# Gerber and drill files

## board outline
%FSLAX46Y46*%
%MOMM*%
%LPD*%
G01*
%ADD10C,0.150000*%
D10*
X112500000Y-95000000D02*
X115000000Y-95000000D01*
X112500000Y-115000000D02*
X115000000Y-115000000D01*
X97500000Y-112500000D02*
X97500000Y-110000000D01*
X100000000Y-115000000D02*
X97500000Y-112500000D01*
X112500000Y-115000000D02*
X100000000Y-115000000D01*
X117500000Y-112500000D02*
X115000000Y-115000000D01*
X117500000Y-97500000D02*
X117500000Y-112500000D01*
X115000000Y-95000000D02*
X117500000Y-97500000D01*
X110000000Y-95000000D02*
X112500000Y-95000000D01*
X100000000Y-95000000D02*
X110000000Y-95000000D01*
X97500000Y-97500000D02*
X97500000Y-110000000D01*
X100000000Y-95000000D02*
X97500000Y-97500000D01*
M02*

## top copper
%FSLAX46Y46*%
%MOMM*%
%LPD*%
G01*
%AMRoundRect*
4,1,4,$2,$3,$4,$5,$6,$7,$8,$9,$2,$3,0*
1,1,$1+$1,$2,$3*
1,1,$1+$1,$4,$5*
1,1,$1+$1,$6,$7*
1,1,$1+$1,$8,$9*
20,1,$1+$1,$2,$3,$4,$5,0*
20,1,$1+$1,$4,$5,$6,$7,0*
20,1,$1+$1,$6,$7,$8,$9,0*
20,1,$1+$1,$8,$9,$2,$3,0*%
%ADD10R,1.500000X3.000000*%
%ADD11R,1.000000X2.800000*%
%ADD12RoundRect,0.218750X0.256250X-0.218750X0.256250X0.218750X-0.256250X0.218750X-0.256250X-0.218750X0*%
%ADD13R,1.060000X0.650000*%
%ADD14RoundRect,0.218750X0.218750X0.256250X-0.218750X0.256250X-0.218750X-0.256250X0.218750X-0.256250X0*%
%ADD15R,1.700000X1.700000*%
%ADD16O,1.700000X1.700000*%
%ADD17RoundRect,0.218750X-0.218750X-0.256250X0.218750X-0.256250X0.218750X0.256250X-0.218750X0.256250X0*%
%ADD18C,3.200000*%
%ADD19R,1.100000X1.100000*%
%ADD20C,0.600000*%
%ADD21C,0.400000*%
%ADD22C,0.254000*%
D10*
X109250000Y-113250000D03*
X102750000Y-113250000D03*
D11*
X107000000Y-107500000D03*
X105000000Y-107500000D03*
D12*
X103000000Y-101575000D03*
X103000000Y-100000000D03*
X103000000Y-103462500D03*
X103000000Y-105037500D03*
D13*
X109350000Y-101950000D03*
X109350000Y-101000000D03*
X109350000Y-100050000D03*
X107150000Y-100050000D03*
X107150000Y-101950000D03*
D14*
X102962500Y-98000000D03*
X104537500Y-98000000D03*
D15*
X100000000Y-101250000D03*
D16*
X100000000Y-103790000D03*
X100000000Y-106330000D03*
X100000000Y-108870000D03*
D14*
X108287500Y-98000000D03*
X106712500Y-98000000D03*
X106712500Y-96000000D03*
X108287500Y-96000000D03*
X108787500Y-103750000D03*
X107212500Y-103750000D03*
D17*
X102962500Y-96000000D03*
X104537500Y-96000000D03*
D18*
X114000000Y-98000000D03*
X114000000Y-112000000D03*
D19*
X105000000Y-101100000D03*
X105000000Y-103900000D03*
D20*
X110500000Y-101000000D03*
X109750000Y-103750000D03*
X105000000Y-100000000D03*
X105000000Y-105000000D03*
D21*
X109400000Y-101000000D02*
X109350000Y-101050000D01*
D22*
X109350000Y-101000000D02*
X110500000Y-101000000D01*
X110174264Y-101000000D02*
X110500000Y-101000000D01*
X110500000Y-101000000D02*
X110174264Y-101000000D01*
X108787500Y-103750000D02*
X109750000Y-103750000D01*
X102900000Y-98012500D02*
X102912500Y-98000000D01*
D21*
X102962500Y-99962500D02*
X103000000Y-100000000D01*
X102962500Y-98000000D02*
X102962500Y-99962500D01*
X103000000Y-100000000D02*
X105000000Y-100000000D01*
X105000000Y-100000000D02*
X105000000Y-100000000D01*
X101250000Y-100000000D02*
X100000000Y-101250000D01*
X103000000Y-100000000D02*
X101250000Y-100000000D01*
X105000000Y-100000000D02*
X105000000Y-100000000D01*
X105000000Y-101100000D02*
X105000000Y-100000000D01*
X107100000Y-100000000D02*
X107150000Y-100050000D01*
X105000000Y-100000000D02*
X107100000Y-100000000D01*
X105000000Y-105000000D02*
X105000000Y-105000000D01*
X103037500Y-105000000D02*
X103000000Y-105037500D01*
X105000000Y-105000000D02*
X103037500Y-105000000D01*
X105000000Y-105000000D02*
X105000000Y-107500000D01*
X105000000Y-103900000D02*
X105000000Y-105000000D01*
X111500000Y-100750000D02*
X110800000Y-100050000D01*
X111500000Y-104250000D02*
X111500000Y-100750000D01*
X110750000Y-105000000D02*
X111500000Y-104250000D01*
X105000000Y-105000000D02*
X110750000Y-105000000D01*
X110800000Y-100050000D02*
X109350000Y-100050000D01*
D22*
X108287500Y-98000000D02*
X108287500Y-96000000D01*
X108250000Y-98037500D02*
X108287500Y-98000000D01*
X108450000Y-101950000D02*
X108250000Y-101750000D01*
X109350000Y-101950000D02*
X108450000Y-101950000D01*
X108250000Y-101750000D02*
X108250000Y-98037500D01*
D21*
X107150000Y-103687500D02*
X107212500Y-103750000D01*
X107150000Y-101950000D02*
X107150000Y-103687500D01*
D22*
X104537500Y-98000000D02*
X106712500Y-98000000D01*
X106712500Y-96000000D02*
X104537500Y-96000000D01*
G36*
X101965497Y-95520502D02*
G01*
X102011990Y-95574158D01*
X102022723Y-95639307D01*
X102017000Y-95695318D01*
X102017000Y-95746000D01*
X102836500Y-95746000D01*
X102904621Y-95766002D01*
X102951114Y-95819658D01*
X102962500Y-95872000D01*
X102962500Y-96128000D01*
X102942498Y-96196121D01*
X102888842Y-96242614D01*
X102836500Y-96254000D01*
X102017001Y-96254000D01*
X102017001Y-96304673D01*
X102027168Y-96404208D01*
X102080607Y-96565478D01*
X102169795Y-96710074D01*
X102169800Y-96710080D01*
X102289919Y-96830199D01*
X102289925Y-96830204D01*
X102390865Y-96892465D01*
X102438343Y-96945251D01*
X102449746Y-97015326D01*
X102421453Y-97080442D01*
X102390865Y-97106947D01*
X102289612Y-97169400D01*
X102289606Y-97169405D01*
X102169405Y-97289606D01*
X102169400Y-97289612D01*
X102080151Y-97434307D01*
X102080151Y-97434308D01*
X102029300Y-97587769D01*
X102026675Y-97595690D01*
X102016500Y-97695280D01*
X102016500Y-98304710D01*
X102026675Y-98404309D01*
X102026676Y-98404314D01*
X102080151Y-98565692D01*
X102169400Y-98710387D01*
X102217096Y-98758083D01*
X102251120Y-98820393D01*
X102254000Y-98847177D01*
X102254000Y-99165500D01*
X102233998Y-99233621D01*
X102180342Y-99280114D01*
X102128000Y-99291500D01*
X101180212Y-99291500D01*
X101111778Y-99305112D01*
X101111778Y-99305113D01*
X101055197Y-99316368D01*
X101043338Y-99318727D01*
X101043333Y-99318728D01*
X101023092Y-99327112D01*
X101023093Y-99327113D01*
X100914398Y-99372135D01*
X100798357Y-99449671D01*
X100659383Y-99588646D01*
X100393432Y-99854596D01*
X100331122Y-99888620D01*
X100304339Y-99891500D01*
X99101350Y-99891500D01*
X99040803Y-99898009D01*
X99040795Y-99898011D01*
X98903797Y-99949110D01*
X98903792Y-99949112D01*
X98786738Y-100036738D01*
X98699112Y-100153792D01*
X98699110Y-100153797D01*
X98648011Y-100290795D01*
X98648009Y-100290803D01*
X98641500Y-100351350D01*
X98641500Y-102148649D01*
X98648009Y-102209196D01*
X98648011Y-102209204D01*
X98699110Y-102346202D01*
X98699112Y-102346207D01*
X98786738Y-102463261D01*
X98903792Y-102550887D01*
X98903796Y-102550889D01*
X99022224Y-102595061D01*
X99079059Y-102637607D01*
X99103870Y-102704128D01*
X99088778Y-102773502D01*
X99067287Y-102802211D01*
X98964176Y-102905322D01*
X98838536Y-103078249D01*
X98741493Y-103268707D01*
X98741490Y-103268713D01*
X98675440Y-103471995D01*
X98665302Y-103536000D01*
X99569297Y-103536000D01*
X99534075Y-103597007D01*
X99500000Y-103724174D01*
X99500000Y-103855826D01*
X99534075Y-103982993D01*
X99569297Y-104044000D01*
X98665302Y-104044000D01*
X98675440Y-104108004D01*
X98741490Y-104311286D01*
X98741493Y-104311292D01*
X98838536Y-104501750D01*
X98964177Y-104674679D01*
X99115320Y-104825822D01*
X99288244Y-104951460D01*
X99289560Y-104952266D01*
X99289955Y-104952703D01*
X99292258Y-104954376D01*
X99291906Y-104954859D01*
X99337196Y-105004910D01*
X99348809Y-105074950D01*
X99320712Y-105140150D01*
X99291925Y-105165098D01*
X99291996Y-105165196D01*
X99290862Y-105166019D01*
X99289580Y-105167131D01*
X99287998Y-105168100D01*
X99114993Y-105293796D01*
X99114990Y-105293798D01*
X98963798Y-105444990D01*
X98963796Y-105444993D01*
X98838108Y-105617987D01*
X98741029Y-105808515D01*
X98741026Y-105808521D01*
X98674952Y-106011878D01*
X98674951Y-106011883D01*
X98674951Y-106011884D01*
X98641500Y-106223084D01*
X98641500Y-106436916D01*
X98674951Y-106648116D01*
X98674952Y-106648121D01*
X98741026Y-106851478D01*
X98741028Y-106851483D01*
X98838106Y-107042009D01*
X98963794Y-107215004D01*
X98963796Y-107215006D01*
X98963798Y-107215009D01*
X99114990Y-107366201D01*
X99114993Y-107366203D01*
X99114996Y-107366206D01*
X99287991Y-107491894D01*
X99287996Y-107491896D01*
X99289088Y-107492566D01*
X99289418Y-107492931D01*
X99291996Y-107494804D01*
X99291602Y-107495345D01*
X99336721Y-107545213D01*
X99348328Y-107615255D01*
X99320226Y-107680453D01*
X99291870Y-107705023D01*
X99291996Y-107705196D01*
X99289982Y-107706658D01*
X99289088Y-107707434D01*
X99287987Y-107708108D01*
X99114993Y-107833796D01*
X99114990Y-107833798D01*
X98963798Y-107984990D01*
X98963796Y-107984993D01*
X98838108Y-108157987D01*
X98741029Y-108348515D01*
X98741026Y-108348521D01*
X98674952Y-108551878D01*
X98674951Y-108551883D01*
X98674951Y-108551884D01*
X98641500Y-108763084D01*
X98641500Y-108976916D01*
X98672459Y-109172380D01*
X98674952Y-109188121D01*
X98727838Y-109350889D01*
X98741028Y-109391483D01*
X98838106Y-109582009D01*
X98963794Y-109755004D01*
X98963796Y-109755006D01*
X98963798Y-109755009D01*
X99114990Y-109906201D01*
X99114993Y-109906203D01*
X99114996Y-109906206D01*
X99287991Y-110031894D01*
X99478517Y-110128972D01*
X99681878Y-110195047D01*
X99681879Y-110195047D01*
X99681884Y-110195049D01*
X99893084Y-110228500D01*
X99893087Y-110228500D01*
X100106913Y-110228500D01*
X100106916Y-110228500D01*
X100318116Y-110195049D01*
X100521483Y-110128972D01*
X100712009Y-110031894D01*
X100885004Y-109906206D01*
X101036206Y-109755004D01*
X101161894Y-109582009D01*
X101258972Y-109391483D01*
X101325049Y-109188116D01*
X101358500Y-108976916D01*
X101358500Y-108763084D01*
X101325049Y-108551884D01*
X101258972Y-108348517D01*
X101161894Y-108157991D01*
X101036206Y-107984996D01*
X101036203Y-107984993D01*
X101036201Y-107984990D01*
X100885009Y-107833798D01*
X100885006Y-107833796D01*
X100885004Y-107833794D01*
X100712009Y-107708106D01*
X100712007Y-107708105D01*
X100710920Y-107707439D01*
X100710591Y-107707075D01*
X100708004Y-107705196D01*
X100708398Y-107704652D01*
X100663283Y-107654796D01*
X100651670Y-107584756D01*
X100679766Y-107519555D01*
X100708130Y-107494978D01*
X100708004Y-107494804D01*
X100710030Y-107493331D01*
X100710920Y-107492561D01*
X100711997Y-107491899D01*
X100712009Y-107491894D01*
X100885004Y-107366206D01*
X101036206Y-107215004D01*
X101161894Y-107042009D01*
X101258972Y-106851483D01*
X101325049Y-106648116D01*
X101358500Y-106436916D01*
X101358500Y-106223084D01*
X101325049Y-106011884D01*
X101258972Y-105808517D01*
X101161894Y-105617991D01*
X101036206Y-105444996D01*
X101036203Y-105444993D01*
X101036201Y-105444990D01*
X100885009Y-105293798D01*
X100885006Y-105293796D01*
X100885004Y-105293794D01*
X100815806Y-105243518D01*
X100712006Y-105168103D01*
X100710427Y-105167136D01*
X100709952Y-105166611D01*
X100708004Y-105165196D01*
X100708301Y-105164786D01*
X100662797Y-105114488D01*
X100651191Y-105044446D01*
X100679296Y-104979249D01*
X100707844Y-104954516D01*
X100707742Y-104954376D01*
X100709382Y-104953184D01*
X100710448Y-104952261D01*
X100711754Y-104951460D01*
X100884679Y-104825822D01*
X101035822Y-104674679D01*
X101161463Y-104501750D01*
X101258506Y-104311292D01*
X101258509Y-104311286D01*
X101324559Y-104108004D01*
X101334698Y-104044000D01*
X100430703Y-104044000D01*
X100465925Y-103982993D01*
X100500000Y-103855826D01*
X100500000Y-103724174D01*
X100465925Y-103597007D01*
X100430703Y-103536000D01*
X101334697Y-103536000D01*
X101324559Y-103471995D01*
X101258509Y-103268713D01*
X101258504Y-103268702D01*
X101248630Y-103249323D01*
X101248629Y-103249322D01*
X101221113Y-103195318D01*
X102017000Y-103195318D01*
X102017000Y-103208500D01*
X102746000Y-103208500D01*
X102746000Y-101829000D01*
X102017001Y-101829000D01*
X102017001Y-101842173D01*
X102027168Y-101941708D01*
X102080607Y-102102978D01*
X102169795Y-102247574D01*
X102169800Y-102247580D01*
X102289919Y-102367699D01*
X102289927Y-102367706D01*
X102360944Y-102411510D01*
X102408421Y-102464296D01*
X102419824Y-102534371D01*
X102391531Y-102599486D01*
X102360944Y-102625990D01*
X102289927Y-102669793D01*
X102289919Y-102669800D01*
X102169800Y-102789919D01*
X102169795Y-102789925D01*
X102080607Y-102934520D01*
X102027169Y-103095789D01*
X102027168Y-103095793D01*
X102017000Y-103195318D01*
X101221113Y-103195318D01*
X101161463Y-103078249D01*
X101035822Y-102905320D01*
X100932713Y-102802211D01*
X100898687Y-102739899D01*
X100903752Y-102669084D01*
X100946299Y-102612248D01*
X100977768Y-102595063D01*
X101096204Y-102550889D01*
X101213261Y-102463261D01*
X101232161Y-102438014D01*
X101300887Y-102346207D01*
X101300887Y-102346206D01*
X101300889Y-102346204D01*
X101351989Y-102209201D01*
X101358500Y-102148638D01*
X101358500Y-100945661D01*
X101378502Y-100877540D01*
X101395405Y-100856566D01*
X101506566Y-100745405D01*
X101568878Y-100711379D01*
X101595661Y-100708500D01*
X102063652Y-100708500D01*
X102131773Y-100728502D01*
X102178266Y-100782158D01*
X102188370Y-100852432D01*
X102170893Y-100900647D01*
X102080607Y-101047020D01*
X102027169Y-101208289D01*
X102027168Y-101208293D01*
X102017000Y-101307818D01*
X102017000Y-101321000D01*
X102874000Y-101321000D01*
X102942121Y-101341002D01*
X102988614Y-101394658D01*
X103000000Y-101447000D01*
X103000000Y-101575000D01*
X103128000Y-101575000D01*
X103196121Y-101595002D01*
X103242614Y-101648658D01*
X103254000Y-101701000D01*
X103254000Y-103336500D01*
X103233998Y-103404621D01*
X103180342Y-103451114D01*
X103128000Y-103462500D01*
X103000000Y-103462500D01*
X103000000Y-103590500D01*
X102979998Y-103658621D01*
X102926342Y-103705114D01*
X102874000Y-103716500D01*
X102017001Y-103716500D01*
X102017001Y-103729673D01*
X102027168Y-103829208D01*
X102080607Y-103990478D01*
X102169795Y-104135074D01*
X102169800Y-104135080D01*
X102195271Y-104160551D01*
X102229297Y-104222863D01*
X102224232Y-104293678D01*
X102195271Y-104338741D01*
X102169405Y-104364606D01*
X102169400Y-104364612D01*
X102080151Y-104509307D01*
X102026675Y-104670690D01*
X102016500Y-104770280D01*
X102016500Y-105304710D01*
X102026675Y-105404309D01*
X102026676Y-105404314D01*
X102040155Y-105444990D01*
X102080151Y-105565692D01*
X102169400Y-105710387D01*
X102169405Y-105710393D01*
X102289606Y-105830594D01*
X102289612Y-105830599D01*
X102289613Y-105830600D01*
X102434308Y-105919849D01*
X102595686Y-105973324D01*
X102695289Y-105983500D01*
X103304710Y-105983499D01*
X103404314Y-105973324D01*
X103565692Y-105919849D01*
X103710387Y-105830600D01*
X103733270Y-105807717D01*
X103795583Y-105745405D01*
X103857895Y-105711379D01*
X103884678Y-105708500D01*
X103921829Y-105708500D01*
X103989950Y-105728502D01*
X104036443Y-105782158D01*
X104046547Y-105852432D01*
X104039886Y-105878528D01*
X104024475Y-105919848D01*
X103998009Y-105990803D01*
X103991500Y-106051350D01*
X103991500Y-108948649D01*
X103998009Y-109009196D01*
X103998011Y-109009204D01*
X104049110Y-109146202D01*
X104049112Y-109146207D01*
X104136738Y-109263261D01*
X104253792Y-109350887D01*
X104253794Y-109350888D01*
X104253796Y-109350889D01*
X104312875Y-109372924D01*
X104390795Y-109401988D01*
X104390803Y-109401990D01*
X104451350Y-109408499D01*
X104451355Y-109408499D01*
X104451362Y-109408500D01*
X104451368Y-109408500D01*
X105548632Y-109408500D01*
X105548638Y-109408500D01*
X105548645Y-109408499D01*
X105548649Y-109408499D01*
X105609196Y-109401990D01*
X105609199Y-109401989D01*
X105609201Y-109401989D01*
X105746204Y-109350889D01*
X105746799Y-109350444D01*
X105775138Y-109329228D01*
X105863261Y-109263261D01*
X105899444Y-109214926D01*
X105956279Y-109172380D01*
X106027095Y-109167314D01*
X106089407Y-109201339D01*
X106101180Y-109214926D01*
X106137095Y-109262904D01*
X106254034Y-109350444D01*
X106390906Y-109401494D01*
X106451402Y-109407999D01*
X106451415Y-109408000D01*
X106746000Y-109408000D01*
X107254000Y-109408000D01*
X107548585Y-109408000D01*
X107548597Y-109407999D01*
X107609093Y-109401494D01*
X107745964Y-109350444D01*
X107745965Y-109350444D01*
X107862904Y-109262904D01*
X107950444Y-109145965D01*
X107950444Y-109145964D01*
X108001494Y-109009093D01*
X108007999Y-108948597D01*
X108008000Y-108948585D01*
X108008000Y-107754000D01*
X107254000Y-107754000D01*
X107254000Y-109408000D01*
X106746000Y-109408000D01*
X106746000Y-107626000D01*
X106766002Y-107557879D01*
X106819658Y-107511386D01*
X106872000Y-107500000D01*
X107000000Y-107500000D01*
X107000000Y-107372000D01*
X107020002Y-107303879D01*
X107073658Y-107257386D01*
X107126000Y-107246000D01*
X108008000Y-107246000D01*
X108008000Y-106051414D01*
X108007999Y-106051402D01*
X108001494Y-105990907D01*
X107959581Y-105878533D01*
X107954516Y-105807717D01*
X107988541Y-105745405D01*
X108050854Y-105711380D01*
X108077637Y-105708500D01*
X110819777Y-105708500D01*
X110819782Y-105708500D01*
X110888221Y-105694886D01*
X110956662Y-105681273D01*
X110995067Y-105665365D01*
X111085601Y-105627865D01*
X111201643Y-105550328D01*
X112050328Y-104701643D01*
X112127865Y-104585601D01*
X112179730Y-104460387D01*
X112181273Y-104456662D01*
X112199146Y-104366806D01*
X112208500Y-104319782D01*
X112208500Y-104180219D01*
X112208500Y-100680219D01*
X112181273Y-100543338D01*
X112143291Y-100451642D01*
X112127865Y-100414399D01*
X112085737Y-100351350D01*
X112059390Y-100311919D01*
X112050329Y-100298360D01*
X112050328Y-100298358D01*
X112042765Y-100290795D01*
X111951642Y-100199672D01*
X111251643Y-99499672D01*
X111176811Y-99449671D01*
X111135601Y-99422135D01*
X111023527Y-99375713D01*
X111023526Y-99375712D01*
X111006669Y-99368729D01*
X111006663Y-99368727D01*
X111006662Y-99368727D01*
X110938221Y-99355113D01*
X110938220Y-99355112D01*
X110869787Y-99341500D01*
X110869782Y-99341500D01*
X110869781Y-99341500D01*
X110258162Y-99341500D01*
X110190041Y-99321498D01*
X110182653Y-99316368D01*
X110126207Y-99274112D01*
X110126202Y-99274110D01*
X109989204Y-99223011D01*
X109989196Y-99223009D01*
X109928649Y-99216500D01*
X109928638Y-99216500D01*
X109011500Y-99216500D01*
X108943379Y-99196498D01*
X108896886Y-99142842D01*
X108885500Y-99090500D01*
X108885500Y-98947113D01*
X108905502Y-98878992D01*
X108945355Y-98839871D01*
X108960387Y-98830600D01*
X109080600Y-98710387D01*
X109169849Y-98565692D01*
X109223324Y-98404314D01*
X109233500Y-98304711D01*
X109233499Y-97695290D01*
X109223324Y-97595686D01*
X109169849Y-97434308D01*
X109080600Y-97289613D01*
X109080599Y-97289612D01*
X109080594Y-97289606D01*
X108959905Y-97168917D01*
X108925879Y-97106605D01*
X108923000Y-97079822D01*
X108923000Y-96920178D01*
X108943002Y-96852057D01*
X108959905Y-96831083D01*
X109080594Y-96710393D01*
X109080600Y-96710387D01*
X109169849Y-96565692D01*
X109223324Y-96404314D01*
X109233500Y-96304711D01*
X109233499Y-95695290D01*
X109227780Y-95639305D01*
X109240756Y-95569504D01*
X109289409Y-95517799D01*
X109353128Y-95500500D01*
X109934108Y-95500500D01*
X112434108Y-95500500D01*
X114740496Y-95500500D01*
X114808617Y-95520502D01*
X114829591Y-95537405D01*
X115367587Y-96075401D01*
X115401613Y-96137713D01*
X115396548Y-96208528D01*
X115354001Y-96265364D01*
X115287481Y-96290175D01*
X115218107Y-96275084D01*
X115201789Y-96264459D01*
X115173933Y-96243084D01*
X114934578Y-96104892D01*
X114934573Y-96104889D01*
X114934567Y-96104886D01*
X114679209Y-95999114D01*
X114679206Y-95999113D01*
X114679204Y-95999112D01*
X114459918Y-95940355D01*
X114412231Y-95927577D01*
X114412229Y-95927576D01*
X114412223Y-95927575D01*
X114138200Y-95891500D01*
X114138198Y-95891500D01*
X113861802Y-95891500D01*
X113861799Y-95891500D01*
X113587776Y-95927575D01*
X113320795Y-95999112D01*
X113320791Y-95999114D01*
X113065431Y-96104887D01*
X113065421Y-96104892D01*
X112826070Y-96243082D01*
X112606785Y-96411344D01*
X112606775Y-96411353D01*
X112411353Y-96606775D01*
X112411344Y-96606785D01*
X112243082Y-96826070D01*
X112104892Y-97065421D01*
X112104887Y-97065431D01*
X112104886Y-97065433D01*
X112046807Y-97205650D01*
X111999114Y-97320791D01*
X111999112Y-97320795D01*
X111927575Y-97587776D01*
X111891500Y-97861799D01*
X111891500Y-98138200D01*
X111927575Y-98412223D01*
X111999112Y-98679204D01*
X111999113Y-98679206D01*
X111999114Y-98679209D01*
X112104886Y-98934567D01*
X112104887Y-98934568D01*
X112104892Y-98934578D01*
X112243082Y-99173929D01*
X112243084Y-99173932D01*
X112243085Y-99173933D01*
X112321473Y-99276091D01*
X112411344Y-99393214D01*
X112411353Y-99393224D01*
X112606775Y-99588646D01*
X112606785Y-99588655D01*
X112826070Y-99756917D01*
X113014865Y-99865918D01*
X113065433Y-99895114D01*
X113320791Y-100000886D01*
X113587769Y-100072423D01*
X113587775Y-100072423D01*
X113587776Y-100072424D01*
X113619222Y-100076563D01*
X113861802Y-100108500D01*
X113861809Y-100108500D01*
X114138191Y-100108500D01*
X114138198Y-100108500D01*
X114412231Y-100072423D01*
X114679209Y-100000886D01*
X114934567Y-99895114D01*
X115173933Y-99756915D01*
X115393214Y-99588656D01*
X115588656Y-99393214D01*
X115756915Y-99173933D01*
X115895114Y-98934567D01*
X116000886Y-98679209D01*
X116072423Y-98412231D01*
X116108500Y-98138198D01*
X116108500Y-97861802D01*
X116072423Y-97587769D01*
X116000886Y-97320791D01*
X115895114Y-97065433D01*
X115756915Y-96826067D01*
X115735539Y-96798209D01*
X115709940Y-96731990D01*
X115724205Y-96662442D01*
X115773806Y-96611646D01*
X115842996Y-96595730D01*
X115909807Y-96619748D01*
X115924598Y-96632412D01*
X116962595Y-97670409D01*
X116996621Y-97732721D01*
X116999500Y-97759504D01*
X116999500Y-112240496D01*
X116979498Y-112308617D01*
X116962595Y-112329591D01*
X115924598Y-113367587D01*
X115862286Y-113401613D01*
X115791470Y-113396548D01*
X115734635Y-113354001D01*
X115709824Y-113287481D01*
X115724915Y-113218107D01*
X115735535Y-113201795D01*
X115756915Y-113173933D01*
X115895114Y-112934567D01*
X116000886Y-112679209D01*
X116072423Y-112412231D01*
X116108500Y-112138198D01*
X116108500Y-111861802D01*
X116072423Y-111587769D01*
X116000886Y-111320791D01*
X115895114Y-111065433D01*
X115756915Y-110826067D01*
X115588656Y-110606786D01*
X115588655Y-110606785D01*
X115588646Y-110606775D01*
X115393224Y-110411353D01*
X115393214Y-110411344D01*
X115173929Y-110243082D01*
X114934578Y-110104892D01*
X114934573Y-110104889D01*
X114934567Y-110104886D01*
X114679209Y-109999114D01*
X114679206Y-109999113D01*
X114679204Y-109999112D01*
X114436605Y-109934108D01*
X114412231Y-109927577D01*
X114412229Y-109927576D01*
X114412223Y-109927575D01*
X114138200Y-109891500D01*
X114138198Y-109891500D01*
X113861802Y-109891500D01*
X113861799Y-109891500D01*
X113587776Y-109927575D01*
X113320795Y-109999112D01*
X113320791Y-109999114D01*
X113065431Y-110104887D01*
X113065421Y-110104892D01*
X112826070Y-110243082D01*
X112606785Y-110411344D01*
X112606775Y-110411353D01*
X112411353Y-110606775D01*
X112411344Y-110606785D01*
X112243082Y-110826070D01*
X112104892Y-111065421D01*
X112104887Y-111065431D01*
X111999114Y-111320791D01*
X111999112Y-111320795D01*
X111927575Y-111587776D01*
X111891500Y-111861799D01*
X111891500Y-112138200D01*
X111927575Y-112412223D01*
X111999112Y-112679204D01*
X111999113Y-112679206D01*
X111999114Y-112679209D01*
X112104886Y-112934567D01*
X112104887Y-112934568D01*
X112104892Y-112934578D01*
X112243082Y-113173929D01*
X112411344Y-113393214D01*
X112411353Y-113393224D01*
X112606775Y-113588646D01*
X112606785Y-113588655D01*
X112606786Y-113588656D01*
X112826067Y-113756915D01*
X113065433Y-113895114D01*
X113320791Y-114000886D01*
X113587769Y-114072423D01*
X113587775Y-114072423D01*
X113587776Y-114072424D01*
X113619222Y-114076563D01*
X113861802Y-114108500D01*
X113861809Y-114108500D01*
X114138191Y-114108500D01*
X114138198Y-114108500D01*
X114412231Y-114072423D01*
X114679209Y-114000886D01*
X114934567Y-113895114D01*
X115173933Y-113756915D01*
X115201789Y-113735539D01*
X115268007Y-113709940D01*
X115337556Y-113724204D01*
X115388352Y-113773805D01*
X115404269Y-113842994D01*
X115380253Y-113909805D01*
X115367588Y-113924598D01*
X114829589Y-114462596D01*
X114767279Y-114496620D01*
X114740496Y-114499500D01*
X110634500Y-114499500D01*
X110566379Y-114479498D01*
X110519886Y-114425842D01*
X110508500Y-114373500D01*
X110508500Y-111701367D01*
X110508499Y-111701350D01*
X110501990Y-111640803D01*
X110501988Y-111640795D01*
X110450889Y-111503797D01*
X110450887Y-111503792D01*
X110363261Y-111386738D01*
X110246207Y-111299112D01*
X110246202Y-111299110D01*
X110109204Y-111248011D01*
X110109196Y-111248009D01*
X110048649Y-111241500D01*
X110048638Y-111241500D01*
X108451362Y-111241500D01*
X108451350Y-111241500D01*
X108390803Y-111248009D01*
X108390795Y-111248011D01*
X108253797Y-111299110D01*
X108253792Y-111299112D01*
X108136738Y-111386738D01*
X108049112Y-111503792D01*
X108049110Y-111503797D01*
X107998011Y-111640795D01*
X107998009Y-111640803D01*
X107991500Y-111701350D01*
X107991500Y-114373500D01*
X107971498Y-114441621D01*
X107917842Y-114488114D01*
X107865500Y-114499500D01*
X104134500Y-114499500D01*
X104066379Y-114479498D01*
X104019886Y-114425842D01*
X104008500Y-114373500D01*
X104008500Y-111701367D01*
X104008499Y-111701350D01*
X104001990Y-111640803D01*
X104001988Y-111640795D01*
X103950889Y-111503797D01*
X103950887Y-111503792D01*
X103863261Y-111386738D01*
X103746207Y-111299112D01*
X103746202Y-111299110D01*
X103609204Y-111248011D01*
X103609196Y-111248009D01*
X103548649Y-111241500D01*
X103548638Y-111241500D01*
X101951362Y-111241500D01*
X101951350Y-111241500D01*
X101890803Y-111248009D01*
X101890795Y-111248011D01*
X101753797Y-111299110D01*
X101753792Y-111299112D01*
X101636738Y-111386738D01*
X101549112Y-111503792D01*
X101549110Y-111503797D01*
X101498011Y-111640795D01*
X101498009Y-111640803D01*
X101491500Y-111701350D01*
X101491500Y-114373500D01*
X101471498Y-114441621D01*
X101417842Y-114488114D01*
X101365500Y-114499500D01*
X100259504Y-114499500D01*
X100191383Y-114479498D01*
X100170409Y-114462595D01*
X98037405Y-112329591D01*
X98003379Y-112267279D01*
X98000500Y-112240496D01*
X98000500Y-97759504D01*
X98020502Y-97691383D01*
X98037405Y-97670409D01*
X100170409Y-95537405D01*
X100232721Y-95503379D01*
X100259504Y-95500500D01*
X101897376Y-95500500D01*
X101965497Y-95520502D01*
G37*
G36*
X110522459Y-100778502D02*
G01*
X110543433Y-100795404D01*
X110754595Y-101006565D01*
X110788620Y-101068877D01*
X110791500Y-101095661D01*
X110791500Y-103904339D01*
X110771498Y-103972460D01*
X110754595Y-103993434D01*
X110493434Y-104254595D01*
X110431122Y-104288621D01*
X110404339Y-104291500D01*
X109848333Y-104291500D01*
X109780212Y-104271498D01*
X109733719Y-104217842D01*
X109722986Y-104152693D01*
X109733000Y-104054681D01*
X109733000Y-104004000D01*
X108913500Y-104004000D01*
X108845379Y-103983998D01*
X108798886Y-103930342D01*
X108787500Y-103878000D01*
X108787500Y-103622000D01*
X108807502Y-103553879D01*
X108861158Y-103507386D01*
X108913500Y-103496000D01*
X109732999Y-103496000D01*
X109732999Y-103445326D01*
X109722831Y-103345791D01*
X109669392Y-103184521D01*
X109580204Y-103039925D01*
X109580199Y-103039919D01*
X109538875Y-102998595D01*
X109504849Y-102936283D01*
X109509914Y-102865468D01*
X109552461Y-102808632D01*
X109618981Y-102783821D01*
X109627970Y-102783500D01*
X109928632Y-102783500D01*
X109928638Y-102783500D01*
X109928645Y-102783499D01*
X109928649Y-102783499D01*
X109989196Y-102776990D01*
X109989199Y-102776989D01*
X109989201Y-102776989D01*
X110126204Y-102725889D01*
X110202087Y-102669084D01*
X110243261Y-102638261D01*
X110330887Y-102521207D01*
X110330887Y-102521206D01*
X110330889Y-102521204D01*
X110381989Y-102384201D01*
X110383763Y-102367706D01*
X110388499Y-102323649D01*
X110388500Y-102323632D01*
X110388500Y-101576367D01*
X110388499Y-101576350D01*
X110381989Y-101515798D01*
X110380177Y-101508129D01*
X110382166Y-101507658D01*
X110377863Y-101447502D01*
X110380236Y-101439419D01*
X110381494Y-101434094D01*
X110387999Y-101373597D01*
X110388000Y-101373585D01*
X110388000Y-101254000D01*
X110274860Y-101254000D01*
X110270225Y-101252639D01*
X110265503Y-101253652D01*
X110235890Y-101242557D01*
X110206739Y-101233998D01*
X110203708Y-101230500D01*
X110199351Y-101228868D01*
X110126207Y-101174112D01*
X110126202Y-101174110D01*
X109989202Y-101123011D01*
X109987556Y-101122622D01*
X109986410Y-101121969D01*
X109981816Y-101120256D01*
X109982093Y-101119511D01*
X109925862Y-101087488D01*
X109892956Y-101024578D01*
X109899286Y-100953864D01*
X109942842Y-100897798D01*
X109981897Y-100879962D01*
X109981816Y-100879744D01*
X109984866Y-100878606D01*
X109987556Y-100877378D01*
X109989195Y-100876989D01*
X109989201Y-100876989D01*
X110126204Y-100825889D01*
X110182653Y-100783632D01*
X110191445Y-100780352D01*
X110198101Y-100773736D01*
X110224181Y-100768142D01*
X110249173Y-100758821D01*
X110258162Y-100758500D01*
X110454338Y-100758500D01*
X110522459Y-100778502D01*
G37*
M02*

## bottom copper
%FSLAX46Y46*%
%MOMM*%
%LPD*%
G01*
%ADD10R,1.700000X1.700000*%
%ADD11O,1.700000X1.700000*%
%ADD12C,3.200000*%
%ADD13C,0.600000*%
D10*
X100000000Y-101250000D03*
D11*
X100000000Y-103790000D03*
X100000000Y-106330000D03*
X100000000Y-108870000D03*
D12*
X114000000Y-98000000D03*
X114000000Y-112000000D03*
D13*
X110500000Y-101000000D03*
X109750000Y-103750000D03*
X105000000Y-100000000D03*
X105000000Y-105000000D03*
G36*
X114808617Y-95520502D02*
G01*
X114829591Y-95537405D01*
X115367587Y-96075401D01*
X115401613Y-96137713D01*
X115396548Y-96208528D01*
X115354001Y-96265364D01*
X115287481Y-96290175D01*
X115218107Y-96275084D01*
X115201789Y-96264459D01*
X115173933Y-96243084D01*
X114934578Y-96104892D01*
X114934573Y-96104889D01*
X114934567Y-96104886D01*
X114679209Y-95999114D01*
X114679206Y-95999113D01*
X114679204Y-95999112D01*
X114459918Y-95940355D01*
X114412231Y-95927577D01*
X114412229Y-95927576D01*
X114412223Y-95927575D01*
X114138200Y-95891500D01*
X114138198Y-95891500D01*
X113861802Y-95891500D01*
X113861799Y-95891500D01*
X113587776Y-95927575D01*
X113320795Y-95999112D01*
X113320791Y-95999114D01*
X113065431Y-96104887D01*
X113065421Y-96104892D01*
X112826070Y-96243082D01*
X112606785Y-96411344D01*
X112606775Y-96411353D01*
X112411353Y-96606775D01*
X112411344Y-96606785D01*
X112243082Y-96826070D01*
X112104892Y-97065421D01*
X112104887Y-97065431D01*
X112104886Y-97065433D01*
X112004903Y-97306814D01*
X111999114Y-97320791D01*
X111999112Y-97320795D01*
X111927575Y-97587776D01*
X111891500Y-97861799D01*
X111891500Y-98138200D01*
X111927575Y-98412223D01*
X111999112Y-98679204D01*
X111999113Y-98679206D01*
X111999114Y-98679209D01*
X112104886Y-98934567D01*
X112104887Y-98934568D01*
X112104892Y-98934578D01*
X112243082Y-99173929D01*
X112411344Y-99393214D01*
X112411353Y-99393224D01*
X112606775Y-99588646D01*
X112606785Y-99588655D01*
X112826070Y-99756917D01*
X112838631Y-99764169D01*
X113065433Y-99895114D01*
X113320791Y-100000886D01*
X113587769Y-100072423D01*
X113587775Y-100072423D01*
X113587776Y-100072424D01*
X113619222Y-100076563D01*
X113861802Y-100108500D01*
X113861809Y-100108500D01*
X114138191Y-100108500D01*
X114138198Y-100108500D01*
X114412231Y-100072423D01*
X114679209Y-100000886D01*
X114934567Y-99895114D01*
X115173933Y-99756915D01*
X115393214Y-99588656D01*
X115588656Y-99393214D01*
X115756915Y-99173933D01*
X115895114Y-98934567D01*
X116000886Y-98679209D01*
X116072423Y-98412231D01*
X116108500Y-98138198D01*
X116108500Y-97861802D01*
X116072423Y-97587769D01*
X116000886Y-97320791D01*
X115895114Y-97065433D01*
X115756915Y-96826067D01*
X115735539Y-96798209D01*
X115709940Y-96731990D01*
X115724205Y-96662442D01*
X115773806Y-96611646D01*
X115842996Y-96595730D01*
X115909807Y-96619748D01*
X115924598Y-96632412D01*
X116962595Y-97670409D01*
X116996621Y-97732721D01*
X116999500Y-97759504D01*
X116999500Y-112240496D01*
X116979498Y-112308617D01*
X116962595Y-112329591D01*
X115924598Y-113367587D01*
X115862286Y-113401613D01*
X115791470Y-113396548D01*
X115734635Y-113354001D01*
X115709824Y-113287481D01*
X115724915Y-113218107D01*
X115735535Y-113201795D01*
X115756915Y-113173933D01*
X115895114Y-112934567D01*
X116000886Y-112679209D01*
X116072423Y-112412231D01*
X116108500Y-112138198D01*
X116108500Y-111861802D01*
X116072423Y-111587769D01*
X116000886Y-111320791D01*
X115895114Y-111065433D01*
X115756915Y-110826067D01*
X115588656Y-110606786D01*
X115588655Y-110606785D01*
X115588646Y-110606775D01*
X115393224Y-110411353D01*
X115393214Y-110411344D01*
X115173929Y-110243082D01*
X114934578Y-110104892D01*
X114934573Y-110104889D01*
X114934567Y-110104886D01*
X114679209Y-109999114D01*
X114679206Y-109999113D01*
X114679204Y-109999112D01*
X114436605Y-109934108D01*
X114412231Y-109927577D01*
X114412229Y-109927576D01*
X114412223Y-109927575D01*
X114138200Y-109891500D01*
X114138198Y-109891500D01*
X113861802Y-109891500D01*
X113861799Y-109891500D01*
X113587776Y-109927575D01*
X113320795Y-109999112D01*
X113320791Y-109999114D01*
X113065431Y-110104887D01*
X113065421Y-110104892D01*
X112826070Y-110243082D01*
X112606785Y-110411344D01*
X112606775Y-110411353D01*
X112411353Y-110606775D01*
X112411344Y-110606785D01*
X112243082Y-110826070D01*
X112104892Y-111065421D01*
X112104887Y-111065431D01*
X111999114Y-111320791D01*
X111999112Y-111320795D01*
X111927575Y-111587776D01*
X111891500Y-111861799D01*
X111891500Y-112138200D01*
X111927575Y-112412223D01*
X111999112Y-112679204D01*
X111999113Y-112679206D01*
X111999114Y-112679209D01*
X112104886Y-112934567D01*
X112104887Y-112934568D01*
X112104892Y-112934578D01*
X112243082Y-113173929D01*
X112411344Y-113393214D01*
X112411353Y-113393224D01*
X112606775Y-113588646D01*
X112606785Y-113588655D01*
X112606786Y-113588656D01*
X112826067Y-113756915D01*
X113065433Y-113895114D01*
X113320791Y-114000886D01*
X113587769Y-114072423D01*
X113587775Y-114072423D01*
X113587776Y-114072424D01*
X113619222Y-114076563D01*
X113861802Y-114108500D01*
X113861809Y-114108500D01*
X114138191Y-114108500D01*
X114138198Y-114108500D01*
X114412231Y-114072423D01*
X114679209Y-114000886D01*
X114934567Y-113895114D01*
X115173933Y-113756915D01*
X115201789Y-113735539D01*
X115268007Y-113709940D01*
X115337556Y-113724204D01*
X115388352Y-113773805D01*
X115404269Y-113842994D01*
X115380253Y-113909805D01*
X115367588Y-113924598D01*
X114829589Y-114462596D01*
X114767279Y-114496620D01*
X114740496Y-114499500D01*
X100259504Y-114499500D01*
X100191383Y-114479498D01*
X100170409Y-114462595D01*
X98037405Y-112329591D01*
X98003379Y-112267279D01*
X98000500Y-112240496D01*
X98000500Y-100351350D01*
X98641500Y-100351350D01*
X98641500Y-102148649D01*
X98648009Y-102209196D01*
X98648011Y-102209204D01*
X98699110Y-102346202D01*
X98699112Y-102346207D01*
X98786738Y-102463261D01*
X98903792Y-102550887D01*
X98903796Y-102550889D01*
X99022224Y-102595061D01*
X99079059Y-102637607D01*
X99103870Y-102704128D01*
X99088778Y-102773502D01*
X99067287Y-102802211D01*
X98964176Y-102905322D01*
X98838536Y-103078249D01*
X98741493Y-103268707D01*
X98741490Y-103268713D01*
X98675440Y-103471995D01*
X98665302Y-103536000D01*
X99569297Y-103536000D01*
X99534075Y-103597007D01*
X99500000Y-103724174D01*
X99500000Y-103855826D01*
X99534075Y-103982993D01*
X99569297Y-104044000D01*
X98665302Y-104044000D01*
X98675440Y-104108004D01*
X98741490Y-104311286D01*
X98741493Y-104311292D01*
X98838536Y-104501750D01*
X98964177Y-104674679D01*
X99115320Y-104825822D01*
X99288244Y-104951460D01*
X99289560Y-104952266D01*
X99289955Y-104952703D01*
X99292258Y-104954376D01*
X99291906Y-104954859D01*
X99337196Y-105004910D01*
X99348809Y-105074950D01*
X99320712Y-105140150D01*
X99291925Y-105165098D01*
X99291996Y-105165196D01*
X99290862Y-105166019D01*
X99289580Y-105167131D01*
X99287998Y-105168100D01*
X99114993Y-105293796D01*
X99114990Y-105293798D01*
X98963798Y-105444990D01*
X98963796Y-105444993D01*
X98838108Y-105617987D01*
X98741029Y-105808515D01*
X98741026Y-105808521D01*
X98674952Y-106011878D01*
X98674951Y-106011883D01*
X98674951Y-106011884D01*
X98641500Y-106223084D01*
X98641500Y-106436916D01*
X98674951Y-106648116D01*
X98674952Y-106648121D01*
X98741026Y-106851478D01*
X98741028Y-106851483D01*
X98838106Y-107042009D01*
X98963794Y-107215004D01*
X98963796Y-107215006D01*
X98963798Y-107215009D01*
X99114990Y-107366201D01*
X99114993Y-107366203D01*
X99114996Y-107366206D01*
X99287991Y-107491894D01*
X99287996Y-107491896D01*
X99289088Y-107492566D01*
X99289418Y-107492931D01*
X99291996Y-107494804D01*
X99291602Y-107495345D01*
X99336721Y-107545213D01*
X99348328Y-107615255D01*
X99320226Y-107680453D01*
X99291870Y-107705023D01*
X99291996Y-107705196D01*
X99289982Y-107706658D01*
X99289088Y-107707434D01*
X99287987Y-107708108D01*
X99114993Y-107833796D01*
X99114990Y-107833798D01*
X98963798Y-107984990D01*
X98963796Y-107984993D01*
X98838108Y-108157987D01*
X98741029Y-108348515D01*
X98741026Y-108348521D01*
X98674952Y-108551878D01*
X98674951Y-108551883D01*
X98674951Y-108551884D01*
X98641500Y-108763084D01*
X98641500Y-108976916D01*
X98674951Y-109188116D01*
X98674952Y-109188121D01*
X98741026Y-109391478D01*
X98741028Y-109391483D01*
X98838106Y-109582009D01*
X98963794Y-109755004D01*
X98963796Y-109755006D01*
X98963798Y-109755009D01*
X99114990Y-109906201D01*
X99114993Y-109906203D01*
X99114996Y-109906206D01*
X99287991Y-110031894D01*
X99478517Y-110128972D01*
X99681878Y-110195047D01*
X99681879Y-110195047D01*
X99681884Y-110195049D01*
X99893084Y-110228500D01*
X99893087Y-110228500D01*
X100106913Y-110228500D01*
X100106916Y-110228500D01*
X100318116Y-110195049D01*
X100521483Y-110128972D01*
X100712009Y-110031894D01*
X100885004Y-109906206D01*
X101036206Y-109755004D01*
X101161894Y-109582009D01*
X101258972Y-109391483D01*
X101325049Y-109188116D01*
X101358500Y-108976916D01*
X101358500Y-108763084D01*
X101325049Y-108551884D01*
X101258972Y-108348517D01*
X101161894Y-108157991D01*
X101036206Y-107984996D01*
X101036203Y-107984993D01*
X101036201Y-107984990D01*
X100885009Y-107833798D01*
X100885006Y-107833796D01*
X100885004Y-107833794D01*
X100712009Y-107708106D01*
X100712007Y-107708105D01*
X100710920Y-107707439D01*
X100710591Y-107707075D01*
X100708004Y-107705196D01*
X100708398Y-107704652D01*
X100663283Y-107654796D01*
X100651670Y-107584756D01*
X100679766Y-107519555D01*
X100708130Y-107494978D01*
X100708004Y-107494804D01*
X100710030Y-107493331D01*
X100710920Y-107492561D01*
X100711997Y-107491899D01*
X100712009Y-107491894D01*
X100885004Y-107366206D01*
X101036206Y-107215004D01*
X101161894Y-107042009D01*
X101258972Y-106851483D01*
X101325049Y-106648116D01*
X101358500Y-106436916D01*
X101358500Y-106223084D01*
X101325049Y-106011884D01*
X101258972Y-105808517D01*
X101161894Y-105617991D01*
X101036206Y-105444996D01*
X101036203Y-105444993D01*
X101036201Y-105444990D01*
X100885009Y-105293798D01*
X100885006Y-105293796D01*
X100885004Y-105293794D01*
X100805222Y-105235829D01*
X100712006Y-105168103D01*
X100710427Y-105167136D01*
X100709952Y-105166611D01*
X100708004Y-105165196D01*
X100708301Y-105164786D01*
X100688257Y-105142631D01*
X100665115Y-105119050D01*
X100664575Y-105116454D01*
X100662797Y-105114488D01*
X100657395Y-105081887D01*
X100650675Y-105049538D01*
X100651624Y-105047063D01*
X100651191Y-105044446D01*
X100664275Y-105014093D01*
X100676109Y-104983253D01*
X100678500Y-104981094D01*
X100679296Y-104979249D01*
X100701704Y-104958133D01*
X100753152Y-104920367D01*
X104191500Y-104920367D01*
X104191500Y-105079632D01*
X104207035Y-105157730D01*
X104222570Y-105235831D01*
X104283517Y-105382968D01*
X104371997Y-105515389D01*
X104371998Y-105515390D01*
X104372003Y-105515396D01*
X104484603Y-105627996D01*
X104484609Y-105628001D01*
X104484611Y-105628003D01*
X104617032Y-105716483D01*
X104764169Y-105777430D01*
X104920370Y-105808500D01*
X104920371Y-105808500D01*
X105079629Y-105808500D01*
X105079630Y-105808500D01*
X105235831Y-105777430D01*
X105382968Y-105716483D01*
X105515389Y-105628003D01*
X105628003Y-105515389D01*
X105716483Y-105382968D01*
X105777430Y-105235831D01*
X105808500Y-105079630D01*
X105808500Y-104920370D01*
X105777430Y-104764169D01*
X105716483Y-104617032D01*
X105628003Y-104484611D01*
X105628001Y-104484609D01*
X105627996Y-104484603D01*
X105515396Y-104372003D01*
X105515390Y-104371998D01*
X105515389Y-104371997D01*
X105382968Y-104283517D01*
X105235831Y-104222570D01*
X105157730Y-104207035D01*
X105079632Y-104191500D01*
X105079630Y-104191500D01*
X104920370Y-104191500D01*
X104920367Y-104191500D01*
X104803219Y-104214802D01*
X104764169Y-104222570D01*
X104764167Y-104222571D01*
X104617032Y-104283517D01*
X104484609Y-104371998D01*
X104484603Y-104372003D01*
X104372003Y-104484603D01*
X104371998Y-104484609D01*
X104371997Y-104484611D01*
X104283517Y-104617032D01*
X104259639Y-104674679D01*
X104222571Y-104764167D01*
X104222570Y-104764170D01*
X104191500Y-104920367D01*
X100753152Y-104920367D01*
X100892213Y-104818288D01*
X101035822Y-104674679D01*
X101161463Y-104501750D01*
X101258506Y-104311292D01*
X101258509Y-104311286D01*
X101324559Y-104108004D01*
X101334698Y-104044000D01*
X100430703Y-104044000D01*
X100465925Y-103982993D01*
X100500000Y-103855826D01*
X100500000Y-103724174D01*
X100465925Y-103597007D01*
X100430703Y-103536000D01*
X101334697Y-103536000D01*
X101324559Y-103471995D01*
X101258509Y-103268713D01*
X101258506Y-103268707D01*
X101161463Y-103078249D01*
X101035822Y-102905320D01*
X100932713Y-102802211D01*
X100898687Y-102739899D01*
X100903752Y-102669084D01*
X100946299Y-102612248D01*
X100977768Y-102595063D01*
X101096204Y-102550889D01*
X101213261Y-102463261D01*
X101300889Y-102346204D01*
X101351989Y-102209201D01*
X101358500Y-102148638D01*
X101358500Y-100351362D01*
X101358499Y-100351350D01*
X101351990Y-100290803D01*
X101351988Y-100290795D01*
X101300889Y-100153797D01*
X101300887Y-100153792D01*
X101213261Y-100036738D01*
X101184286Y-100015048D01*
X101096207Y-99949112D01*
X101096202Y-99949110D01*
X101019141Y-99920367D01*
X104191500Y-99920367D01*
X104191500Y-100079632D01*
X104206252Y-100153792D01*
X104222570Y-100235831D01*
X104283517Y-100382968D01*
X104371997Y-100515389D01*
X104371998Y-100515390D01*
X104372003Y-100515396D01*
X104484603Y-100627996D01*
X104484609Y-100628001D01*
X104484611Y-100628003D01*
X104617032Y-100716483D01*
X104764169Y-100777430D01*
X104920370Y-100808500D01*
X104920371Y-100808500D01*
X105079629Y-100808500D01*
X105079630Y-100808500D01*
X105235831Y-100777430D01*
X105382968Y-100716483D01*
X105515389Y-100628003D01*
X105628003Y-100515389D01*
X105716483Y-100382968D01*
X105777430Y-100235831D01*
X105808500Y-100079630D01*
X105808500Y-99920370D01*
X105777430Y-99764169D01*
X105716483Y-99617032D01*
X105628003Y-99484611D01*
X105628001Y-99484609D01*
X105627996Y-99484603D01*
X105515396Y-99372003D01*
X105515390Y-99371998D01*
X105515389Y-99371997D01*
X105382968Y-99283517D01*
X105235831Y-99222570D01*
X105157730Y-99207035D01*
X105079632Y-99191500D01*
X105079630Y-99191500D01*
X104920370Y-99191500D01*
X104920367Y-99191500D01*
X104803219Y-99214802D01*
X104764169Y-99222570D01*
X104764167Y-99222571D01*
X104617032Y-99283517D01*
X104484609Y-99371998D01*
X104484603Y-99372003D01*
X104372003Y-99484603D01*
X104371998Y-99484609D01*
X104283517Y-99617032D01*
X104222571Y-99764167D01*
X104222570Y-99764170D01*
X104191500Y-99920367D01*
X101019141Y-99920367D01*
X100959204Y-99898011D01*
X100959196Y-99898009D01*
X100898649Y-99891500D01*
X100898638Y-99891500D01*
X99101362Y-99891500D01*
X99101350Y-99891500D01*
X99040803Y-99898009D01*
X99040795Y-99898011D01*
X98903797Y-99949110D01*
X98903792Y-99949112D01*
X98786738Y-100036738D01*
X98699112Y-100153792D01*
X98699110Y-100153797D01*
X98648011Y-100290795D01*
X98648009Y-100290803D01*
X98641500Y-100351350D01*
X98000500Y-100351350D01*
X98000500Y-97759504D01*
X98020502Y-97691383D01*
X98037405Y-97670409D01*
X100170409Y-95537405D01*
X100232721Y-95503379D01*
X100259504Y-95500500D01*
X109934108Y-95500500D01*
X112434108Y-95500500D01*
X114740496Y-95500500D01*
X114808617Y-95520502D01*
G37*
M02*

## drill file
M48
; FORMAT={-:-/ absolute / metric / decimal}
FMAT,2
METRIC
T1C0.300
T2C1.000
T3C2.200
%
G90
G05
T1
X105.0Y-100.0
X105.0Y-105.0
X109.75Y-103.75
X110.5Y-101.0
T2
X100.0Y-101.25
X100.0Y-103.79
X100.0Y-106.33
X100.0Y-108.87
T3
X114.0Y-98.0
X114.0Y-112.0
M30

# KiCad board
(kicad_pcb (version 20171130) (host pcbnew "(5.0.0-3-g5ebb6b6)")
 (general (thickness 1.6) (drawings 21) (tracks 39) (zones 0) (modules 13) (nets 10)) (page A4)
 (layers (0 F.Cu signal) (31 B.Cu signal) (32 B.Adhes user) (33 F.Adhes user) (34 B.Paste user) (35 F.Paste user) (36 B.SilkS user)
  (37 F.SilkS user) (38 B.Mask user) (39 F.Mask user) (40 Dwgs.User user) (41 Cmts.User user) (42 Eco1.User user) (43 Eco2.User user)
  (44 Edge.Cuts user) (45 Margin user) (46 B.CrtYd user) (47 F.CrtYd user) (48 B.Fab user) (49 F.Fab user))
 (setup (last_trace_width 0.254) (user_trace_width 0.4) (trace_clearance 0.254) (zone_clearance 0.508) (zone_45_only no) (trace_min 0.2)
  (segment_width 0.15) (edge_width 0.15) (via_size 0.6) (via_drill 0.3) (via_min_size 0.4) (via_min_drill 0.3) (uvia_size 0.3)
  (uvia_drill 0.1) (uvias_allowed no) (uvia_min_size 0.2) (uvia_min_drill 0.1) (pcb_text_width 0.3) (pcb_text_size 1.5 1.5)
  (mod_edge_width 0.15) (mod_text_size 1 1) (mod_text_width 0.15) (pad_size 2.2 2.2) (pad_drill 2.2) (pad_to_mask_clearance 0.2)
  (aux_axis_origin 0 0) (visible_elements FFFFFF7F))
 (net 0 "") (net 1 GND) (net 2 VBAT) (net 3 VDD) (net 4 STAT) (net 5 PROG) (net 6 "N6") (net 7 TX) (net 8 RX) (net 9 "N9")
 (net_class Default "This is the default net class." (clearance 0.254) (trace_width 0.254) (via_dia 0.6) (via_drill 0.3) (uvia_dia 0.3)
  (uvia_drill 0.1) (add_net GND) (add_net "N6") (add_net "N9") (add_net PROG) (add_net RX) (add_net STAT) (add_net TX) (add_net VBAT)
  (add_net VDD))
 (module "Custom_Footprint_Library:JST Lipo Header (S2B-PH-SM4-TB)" (layer F.Cu) (at 106 112)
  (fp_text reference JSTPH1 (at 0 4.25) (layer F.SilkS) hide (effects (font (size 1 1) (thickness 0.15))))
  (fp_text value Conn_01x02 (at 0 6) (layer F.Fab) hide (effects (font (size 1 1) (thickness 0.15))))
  (pad "" connect rect (at 3.25 1.25) (size 1.5 3) (layers F.Cu F.Mask))
  (pad "" connect rect (at -3.25 1.25) (size 1.5 3) (layers F.Cu F.Mask))
  (pad 2 smd rect (at 1 -4.5) (size 1 2.8) (layers F.Cu F.Paste F.Mask) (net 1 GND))
  (pad 1 smd rect (at -1 -4.5) (size 1 2.8) (layers F.Cu F.Paste F.Mask) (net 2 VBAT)))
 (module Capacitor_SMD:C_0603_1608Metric (layer F.Cu) (at 103 100.7875 90)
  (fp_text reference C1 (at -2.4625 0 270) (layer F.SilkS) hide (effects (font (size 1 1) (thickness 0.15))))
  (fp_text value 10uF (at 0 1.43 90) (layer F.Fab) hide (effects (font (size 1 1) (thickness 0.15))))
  (pad 1 smd roundrect (at -0.7875 0 90) (size 0.875 0.95) (layers F.Cu F.Paste F.Mask) (roundrect_rratio 0.25) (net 1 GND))
  (pad 2 smd roundrect (at 0.7875 0 90) (size 0.875 0.95) (layers F.Cu F.Paste F.Mask) (roundrect_rratio 0.25) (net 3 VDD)))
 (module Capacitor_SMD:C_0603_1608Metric (layer F.Cu) (at 103 104.25 90)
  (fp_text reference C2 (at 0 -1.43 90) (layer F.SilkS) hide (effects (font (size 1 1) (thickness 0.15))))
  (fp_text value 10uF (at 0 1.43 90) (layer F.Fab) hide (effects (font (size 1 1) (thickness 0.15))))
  (pad 2 smd roundrect (at 0.7875 0 90) (size 0.875 0.95) (layers F.Cu F.Paste F.Mask) (roundrect_rratio 0.25) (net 1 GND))
  (pad 1 smd roundrect (at -0.7875 0 90) (size 0.875 0.95) (layers F.Cu F.Paste F.Mask) (roundrect_rratio 0.25) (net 2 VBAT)))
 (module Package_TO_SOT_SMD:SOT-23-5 (layer F.Cu) (at 108.25 101 180)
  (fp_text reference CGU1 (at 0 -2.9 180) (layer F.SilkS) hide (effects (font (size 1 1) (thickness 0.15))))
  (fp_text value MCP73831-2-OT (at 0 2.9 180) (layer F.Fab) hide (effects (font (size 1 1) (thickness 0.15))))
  (pad 1 smd rect (at -1.1 -0.95 180) (size 1.06 0.65) (layers F.Cu F.Paste F.Mask) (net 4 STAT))
  (pad 2 smd rect (at -1.1 0 180) (size 1.06 0.65) (layers F.Cu F.Paste F.Mask) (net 1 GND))
  (pad 3 smd rect (at -1.1 0.95 180) (size 1.06 0.65) (layers F.Cu F.Paste F.Mask) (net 2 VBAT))
  (pad 4 smd rect (at 1.1 0.95 180) (size 1.06 0.65) (layers F.Cu F.Paste F.Mask) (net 3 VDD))
  (pad 5 smd rect (at 1.1 -0.95 180) (size 1.06 0.65) (layers F.Cu F.Paste F.Mask) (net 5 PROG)))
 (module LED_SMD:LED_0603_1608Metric (layer F.Cu) (at 103.75 98 180)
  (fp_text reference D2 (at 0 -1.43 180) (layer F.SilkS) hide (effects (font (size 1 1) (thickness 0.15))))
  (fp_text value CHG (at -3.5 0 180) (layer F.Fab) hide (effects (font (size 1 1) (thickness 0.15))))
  (pad 2 smd roundrect (at 0.7875 0 180) (size 0.875 0.95) (layers F.Cu F.Paste F.Mask) (roundrect_rratio 0.25) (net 3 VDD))
  (pad 1 smd roundrect (at -0.7875 0 180) (size 0.875 0.95) (layers F.Cu F.Paste F.Mask) (roundrect_rratio 0.25) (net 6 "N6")))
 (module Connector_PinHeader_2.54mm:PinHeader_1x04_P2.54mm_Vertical (layer F.Cu) (at 100 101.25)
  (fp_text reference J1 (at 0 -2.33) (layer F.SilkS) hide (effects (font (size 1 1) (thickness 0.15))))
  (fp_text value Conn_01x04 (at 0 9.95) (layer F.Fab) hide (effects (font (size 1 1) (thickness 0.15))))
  (pad 1 thru_hole rect (at 0 0) (size 1.7 1.7) (drill 1) (layers *.Cu *.Mask) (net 3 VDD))
  (pad 2 thru_hole oval (at 0 2.54) (size 1.7 1.7) (drill 1) (layers *.Cu *.Mask) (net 1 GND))
  (pad 3 thru_hole oval (at 0 5.08) (size 1.7 1.7) (drill 1) (layers *.Cu *.Mask) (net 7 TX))
  (pad 4 thru_hole oval (at 0 7.62) (size 1.7 1.7) (drill 1) (layers *.Cu *.Mask) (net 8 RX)))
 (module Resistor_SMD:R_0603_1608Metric (layer F.Cu) (at 107.5 98 180)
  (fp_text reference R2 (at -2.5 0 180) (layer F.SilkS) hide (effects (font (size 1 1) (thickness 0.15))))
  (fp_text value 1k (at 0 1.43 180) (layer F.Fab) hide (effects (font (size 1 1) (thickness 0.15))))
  (pad 1 smd roundrect (at -0.7875 0 180) (size 0.875 0.95) (layers F.Cu F.Paste F.Mask) (roundrect_rratio 0.25) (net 4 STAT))
  (pad 2 smd roundrect (at 0.7875 0 180) (size 0.875 0.95) (layers F.Cu F.Paste F.Mask) (roundrect_rratio 0.25) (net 6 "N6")))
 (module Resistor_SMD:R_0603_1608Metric (layer F.Cu) (at 107.5 96 180)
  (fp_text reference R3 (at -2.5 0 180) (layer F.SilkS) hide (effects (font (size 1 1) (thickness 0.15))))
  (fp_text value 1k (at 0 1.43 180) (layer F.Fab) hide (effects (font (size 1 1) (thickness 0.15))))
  (pad 2 smd roundrect (at 0.7875 0 180) (size 0.875 0.95) (layers F.Cu F.Paste F.Mask) (roundrect_rratio 0.25) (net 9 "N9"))
  (pad 1 smd roundrect (at -0.7875 0 180) (size 0.875 0.95) (layers F.Cu F.Paste F.Mask) (roundrect_rratio 0.25) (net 4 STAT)))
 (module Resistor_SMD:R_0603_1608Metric (layer F.Cu) (at 108 103.75 180)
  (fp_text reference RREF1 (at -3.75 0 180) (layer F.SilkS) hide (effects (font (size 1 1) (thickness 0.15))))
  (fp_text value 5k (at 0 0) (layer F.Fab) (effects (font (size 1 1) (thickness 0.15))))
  (pad 1 smd roundrect (at -0.7875 0 180) (size 0.875 0.95) (layers F.Cu F.Paste F.Mask) (roundrect_rratio 0.25) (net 1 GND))
  (pad 2 smd roundrect (at 0.7875 0 180) (size 0.875 0.95) (layers F.Cu F.Paste F.Mask) (roundrect_rratio 0.25) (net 5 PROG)))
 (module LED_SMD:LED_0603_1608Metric (layer F.Cu) (at 103.75 96)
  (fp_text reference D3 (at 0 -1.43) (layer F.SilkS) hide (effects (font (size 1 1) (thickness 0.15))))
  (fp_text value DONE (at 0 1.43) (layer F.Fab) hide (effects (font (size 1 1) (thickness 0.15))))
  (pad 1 smd roundrect (at -0.7875 0) (size 0.875 0.95) (layers F.Cu F.Paste F.Mask) (roundrect_rratio 0.25) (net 1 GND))
  (pad 2 smd roundrect (at 0.7875 0) (size 0.875 0.95) (layers F.Cu F.Paste F.Mask) (roundrect_rratio 0.25) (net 9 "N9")))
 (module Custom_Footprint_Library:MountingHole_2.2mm (layer F.Cu) (at 114 98)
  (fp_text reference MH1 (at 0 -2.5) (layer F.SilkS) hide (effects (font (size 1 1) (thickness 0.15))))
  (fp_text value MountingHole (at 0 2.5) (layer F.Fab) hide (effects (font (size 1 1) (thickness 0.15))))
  (pad "" thru_hole circle (at 0 0) (size 3.2 3.2) (drill 2.2) (layers *.Cu *.Mask)))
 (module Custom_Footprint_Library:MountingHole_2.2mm (layer F.Cu) (at 114 112)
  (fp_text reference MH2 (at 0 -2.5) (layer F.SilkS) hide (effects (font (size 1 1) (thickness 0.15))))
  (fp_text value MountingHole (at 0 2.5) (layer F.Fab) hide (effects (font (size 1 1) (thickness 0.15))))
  (pad "" thru_hole circle (at 0 0) (size 3.2 3.2) (drill 2.2) (layers *.Cu *.Mask)))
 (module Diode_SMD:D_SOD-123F (layer F.Cu) (at 105 102.5 270)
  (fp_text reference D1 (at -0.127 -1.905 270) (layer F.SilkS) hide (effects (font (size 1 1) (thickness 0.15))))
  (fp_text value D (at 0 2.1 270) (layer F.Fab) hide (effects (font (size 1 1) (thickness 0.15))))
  (pad 1 smd rect (at -1.4 0 270) (size 1.1 1.1) (layers F.Cu F.Paste F.Mask) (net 3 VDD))
  (pad 2 smd rect (at 1.4 0 270) (size 1.1 1.1) (layers F.Cu F.Paste F.Mask) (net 2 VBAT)))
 (gr_line (start 112.5 95) (end 115 95) (layer Edge.Cuts) (width 0.15))
 (gr_line (start 112.5 115) (end 115 115) (layer Edge.Cuts) (width 0.15))
 (gr_line (start 97.5 112.5) (end 97.5 110) (layer Edge.Cuts) (width 0.15))
 (gr_line (start 100 115) (end 97.5 112.5) (layer Edge.Cuts) (width 0.15))
 (gr_line (start 112.5 115) (end 100 115) (layer Edge.Cuts) (width 0.15))
 (gr_line (start 117.5 112.5) (end 115 115) (layer Edge.Cuts) (width 0.15))
 (gr_line (start 117.5 97.5) (end 117.5 112.5) (layer Edge.Cuts) (width 0.15))
 (gr_line (start 115 95) (end 117.5 97.5) (layer Edge.Cuts) (width 0.15))
 (gr_line (start 110 95) (end 112.5 95) (layer Edge.Cuts) (width 0.15))
 (gr_line (start 100 95) (end 110 95) (layer Edge.Cuts) (width 0.15))
 (gr_line (start 97.5 97.5) (end 97.5 110) (layer Edge.Cuts) (width 0.15))
 (gr_line (start 100 95) (end 97.5 97.5) (layer Edge.Cuts) (width 0.15))
 (segment (start 109.4 101) (end 109.35 101.05) (width 0.4) (layer F.Cu) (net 1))
 (segment (start 109.35 101) (end 110.5 101) (width 0.254) (layer F.Cu) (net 1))
 (segment (start 110.174264 101) (end 110.5 101) (width 0.254) (layer F.Cu) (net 1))
 (segment (start 110.5 101) (end 110.174264 101) (width 0.254) (layer F.Cu) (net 1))
 (via (at 110.5 101) (size 0.6) (drill 0.3) (layers F.Cu B.Cu) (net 1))
 (segment (start 108.7875 103.75) (end 109.75 103.75) (width 0.254) (layer F.Cu) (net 1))
 (via (at 109.75 103.75) (size 0.6) (drill 0.3) (layers F.Cu B.Cu) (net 1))
 (segment (start 102.9 98.0125) (end 102.9125 98) (width 0.254) (layer F.Cu) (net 3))
 (segment (start 102.9625 99.9625) (end 103 100) (width 0.4) (layer F.Cu) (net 3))
 (segment (start 102.9625 98) (end 102.9625 99.9625) (width 0.4) (layer F.Cu) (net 3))
 (segment (start 103 100) (end 105 100) (width 0.4) (layer F.Cu) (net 3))
 (segment (start 105 100) (end 105 100) (width 0.4) (layer F.Cu) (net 3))
 (segment (start 101.25 100) (end 100 101.25) (width 0.4) (layer F.Cu) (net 3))
 (segment (start 103 100) (end 101.25 100) (width 0.4) (layer F.Cu) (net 3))
 (segment (start 105 100) (end 105 100) (width 0.4) (layer F.Cu) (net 3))
 (via (at 105 100) (size 0.6) (drill 0.3) (layers F.Cu B.Cu) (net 3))
 (segment (start 105 101.1) (end 105 100) (width 0.4) (layer F.Cu) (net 3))
 (segment (start 107.1 100) (end 107.15 100.05) (width 0.4) (layer F.Cu) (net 3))
 (segment (start 105 100) (end 107.1 100) (width 0.4) (layer F.Cu) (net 3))
 (segment (start 105 105) (end 105 105) (width 0.4) (layer F.Cu) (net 2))
 (via (at 105 105) (size 0.6) (drill 0.3) (layers F.Cu B.Cu) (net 2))
 (segment (start 103.0375 105) (end 103 105.0375) (width 0.4) (layer F.Cu) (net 2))
 (segment (start 105 105) (end 103.0375 105) (width 0.4) (layer F.Cu) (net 2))
 (segment (start 105 105) (end 105 107.5) (width 0.4) (layer F.Cu) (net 2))
 (segment (start 105 103.9) (end 105 105) (width 0.4) (layer F.Cu) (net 2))
 (segment (start 111.5 100.75) (end 110.8 100.05) (width 0.4) (layer F.Cu) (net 2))
 (segment (start 111.5 104.25) (end 111.5 100.75) (width 0.4) (layer F.Cu) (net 2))
 (segment (start 110.75 105) (end 111.5 104.25) (width 0.4) (layer F.Cu) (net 2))
 (segment (start 105 105) (end 110.75 105) (width 0.4) (layer F.Cu) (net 2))
 (segment (start 110.8 100.05) (end 109.35 100.05) (width 0.4) (layer F.Cu) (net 2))
 (segment (start 108.2875 98) (end 108.2875 96) (width 0.254) (layer F.Cu) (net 4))
 (segment (start 108.25 98.0375) (end 108.2875 98) (width 0.254) (layer F.Cu) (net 4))
 (segment (start 108.45 101.95) (end 108.25 101.75) (width 0.254) (layer F.Cu) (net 4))
 (segment (start 109.35 101.95) (end 108.45 101.95) (width 0.254) (layer F.Cu) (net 4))
 (segment (start 108.25 101.75) (end 108.25 98.0375) (width 0.254) (layer F.Cu) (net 4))
 (segment (start 107.15 103.6875) (end 107.2125 103.75) (width 0.4) (layer F.Cu) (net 5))
 (segment (start 107.15 101.95) (end 107.15 103.6875) (width 0.4) (layer F.Cu) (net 5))
 (segment (start 104.5375 98) (end 106.7125 98) (width 0.254) (layer F.Cu) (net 6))
 (segment (start 106.7125 96) (end 104.5375 96) (width 0.254) (layer F.Cu) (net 9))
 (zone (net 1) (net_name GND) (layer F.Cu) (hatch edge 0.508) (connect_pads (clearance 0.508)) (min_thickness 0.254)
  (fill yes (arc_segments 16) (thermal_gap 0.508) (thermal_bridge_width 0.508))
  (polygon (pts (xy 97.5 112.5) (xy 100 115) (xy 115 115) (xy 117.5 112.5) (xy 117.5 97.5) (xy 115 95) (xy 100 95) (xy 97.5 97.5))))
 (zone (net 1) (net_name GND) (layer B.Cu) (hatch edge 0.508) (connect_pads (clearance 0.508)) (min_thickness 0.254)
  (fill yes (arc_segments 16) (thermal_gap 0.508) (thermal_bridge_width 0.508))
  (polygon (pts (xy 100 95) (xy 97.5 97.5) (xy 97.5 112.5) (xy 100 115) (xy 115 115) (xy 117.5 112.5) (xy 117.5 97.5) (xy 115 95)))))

